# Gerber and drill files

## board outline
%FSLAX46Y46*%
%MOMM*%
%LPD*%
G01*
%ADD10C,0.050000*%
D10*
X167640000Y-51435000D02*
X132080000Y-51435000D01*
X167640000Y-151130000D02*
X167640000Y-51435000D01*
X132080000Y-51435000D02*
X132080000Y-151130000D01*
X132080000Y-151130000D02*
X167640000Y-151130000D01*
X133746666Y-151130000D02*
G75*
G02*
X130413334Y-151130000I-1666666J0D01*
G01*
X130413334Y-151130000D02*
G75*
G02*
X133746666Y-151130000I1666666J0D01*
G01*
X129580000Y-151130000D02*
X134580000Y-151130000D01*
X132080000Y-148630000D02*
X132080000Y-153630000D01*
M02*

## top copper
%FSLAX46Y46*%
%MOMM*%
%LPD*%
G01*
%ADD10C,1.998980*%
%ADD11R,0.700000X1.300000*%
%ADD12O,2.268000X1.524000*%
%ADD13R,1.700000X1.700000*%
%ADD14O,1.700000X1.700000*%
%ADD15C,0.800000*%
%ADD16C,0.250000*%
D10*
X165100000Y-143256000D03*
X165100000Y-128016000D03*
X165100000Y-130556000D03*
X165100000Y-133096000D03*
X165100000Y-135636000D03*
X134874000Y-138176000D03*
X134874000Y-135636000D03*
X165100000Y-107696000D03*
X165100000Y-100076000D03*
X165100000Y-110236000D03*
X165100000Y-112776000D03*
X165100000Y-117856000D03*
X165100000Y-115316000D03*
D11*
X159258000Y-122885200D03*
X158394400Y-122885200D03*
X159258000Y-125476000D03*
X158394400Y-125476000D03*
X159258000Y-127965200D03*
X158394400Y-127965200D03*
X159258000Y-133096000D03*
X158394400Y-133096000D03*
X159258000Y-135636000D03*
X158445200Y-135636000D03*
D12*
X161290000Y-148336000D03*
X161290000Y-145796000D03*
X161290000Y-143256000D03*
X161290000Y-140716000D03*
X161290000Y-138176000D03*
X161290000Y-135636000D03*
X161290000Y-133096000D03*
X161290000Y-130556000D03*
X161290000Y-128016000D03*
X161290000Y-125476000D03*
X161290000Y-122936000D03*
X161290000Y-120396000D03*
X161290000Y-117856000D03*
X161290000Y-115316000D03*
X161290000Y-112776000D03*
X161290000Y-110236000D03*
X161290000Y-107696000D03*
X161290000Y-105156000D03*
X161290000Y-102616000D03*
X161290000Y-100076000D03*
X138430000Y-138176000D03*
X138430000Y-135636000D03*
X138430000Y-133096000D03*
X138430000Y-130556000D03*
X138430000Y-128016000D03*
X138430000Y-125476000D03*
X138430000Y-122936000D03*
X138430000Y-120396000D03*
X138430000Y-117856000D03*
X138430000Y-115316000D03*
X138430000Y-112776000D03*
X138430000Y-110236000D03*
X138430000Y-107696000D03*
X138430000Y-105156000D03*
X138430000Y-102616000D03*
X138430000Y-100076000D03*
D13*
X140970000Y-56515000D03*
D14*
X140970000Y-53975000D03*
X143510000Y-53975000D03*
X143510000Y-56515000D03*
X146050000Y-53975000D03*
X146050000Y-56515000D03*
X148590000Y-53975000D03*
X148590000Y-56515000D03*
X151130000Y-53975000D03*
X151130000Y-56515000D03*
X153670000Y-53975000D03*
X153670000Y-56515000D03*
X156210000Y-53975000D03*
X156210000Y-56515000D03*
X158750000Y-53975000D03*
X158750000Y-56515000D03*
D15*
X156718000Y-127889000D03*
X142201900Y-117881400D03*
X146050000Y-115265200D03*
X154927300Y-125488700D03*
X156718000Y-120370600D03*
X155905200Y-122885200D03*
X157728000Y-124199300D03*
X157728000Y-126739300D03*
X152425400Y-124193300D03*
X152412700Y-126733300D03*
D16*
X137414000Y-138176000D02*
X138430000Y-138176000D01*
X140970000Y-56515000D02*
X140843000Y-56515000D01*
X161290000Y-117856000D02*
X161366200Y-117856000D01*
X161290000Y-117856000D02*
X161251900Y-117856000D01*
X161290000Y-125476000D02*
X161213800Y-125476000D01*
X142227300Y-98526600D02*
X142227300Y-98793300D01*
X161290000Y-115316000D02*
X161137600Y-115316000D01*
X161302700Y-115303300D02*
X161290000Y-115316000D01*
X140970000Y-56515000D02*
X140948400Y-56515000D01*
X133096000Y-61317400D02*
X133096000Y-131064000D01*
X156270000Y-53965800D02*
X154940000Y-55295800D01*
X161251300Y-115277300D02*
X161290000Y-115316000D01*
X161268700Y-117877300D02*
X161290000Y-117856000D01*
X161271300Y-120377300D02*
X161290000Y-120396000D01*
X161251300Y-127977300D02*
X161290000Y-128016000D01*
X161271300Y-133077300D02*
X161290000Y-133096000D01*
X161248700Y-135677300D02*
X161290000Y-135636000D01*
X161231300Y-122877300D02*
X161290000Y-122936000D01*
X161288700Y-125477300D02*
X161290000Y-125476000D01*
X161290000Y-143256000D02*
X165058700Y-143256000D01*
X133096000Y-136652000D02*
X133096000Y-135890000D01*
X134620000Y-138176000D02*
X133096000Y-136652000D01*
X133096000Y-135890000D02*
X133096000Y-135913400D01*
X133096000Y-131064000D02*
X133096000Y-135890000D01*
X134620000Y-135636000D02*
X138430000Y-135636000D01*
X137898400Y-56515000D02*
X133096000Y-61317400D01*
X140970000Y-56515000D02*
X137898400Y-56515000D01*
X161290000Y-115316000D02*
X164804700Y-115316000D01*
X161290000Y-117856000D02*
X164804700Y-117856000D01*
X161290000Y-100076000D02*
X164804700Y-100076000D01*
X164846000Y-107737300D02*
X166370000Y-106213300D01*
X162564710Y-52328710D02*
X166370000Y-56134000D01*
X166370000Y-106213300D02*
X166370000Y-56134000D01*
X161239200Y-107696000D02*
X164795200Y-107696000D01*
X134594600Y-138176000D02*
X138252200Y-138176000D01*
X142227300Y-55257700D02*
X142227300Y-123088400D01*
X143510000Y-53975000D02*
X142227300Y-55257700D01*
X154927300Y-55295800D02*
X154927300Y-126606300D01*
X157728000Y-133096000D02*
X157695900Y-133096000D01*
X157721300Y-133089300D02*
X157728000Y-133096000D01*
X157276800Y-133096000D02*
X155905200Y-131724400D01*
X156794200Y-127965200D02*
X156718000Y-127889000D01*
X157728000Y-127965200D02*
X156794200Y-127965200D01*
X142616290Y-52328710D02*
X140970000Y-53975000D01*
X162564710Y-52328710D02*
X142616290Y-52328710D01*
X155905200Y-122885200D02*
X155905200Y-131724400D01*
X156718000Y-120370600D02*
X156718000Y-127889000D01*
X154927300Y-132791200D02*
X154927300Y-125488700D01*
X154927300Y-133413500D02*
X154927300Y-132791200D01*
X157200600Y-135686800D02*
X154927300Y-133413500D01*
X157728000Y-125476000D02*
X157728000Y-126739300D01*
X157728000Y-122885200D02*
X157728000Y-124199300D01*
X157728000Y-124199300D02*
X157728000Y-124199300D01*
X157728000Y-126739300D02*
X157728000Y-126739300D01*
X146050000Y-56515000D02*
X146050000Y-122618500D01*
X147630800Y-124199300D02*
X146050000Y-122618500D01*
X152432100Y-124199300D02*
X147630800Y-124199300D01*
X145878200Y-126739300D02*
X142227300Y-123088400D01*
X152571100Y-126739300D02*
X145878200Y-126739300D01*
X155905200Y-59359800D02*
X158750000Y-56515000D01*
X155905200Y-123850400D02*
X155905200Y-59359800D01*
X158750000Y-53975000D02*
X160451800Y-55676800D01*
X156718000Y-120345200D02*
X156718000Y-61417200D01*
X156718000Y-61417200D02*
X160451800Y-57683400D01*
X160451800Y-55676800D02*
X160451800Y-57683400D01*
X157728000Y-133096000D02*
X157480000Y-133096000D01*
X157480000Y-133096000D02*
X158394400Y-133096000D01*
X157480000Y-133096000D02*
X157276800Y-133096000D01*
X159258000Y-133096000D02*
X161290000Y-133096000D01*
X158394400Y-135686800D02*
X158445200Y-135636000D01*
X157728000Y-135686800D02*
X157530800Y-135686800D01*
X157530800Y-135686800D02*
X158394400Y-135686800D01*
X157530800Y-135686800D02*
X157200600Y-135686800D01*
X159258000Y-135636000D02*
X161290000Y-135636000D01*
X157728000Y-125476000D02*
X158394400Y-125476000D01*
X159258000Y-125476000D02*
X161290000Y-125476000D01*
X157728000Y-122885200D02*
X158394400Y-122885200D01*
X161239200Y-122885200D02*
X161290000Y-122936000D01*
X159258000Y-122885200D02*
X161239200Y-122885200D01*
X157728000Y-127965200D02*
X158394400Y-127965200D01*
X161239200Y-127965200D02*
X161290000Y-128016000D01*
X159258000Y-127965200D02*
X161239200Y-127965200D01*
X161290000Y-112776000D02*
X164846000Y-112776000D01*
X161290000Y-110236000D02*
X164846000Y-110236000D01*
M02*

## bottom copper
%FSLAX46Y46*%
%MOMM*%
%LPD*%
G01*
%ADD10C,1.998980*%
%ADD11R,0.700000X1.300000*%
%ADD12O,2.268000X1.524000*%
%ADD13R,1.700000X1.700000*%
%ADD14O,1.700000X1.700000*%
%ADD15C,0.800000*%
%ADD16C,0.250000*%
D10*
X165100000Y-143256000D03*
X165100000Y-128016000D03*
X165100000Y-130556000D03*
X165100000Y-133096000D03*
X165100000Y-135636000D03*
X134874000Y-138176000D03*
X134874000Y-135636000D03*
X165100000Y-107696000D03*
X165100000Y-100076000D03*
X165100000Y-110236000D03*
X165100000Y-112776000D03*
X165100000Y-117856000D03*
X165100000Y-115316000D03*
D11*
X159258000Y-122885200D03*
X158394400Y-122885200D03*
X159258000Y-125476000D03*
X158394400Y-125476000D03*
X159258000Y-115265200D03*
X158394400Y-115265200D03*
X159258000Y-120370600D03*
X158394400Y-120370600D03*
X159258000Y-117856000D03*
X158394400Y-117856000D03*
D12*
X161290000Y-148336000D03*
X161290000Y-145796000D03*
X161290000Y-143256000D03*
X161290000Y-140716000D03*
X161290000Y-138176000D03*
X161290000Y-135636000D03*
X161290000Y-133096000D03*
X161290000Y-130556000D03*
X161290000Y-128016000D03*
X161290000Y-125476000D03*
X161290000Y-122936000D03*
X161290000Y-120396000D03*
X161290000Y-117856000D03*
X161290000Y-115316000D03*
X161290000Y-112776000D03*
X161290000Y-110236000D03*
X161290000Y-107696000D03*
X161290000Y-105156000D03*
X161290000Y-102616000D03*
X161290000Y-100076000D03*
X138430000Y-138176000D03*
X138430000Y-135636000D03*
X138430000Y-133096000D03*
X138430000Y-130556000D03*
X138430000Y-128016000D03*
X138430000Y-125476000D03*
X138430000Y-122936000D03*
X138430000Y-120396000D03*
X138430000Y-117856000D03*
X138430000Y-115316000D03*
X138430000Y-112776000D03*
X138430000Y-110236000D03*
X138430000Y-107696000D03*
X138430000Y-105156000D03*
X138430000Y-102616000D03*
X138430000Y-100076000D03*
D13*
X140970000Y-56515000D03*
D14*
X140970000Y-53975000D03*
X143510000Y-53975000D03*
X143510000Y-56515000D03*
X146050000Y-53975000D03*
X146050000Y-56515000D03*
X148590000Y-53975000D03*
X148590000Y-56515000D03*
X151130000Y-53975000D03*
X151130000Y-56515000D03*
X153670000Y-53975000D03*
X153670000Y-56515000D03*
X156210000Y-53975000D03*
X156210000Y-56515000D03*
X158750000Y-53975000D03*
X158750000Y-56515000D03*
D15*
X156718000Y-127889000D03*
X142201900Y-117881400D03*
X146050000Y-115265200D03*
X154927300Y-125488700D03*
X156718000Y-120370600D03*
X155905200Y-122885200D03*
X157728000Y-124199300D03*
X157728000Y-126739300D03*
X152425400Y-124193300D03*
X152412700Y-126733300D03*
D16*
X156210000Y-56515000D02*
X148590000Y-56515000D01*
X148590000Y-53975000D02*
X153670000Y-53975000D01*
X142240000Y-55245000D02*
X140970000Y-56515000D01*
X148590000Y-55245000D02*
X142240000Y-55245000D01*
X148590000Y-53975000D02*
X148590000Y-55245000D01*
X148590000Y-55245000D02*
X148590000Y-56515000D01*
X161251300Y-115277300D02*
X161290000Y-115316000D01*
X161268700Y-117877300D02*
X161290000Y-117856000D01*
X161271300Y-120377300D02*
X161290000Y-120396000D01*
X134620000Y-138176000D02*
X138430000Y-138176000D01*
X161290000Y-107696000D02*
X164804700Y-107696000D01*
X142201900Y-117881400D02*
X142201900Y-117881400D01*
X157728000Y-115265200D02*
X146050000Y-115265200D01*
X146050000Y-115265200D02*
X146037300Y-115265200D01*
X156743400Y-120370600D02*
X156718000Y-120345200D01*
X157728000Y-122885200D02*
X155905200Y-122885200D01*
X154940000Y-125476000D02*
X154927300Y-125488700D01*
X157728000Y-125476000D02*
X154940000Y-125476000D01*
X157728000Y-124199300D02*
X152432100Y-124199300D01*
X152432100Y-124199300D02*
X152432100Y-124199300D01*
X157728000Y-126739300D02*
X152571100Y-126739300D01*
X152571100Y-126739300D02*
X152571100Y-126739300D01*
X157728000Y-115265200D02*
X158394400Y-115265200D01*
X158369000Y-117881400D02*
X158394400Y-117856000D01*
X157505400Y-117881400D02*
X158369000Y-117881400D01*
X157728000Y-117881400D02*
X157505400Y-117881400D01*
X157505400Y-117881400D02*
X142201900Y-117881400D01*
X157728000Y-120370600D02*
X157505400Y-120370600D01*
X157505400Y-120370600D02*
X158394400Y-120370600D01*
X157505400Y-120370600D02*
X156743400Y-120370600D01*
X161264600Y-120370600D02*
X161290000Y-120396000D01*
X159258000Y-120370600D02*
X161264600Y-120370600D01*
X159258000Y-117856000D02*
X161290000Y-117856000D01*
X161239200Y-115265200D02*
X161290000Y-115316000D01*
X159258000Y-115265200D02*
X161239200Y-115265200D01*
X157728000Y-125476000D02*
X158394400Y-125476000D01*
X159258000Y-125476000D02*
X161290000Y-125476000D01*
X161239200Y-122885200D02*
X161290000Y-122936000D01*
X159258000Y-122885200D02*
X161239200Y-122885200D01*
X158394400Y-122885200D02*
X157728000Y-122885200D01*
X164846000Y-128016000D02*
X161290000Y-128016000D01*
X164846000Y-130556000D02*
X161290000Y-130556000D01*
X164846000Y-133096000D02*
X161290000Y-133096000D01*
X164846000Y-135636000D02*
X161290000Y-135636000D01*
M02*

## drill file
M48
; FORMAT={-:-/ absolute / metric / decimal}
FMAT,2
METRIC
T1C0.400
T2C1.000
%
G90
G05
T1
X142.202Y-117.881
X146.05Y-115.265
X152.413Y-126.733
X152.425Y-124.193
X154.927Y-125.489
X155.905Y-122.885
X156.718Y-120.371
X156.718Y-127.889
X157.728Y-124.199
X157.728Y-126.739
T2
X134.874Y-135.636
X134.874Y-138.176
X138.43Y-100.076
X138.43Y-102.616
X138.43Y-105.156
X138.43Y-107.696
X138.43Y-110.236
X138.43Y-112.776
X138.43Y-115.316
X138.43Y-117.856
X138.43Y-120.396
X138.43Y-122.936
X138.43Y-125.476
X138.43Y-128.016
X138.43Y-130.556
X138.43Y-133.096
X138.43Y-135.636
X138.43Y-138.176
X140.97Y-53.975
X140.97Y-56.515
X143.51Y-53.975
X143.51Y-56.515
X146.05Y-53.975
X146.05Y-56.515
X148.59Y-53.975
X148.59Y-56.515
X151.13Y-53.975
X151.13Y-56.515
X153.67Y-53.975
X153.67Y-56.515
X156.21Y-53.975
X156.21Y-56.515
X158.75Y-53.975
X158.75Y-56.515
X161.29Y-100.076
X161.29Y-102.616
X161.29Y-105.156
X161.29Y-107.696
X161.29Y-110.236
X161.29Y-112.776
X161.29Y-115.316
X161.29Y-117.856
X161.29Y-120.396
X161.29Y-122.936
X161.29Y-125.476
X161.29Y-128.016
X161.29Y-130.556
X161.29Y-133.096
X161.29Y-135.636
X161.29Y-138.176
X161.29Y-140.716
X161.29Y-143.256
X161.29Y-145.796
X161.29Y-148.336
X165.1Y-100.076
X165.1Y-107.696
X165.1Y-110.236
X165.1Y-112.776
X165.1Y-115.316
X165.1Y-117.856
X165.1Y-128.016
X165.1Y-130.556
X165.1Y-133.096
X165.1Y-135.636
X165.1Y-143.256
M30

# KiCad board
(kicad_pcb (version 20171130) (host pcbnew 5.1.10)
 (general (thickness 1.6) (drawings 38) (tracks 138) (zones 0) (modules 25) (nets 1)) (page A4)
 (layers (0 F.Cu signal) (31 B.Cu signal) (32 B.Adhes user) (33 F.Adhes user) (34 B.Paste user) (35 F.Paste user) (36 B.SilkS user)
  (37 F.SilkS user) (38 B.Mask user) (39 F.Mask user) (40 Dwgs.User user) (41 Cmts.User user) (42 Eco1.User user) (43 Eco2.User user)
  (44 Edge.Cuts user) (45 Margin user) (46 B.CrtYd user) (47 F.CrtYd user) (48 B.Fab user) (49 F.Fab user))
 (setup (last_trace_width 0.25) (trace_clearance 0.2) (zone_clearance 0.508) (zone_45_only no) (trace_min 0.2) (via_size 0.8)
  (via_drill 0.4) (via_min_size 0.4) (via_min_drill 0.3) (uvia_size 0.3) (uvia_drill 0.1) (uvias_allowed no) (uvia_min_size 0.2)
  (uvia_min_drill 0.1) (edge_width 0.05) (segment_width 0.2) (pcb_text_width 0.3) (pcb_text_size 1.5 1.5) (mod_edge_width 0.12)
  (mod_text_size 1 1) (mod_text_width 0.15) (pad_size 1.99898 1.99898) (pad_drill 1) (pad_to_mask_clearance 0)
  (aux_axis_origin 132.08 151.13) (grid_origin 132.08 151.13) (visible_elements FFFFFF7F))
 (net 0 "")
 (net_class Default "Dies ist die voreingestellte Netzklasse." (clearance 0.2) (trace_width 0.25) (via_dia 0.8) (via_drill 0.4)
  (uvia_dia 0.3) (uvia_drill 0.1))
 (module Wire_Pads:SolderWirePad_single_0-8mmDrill (layer F.Cu) (at 165.1 143.256)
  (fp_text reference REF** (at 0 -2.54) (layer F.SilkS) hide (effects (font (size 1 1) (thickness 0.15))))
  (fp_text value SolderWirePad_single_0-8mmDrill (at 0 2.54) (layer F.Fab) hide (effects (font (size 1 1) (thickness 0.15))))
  (pad 1 thru_hole circle (at 0 0) (size 1.99898 1.99898) (drill 1) (layers *.Cu *.Mask)))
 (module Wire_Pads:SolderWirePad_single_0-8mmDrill (layer F.Cu) (at 165.1 128.016)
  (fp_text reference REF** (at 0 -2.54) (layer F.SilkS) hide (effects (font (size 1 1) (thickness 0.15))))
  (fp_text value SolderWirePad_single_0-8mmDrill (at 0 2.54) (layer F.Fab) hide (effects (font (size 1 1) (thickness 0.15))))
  (pad 1 thru_hole circle (at 0 0) (size 1.99898 1.99898) (drill 1) (layers *.Cu *.Mask)))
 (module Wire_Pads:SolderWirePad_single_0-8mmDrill (layer F.Cu) (at 165.1 130.556)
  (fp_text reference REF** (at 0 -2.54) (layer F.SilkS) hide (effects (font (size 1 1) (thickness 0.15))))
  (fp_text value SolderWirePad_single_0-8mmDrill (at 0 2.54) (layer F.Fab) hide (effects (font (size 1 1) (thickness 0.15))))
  (pad 1 thru_hole circle (at 0 0) (size 1.99898 1.99898) (drill 1) (layers *.Cu *.Mask)))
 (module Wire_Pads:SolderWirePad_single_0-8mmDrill (layer F.Cu) (at 165.1 133.096)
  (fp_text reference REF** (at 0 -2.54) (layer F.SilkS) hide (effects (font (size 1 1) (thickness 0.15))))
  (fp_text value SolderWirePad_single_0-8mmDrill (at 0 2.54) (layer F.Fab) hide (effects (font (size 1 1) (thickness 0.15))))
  (pad 1 thru_hole circle (at 0 0) (size 1.99898 1.99898) (drill 1) (layers *.Cu *.Mask)))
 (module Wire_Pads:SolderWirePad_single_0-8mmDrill (layer F.Cu) (at 165.1 135.636)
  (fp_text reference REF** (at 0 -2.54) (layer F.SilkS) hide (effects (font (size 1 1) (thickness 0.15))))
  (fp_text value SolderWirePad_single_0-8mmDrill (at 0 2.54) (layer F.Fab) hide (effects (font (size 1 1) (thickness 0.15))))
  (pad 1 thru_hole circle (at 0 0) (size 1.99898 1.99898) (drill 1) (layers *.Cu *.Mask)))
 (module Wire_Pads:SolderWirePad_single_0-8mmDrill (layer F.Cu) (at 134.874 138.176)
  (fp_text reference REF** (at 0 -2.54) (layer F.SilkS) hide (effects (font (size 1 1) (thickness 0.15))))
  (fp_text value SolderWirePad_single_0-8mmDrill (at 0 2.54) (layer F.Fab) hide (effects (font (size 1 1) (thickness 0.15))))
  (pad 1 thru_hole circle (at 0 0) (size 1.99898 1.99898) (drill 1) (layers *.Cu *.Mask)))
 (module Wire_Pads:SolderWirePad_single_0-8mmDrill (layer F.Cu) (at 134.874 135.636)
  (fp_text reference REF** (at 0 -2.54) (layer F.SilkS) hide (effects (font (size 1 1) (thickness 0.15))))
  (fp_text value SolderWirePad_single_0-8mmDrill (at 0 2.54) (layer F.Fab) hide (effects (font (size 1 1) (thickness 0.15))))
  (pad 1 thru_hole circle (at 0 0) (size 1.99898 1.99898) (drill 1) (layers *.Cu *.Mask)))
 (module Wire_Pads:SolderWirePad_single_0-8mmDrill (layer F.Cu) (at 165.1 107.696)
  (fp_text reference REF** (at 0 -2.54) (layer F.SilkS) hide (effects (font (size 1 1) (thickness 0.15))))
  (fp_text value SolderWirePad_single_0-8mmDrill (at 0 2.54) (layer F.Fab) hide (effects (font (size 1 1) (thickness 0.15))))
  (pad 1 thru_hole circle (at 0 0) (size 1.99898 1.99898) (drill 1) (layers *.Cu *.Mask)))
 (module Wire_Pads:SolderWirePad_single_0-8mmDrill (layer F.Cu) (at 165.1 100.076)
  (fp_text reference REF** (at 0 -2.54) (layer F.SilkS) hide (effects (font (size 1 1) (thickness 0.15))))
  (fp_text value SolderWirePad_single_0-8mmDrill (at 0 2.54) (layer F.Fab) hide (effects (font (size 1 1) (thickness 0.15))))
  (pad 1 thru_hole circle (at 0 0) (size 1.99898 1.99898) (drill 1) (layers *.Cu *.Mask)))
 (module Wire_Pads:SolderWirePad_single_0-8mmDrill (layer F.Cu) (at 165.1 110.236)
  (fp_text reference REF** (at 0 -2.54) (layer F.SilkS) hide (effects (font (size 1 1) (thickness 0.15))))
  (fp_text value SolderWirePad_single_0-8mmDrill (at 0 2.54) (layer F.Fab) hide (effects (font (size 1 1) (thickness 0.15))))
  (pad 1 thru_hole circle (at 0 0) (size 1.99898 1.99898) (drill 1) (layers *.Cu *.Mask)))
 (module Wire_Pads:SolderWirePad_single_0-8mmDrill (layer F.Cu) (at 165.1 112.776)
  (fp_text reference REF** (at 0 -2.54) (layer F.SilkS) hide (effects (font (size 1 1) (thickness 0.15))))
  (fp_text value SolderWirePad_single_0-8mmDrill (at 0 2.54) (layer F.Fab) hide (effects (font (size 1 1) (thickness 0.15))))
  (pad 1 thru_hole circle (at 0 0) (size 1.99898 1.99898) (drill 1) (layers *.Cu *.Mask)))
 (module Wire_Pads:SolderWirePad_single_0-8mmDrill (layer F.Cu) (at 165.1 117.856)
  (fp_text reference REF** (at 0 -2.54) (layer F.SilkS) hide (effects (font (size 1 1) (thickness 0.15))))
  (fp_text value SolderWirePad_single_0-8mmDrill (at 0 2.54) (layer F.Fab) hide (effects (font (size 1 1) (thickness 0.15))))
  (pad 1 thru_hole circle (at 0 0) (size 1.99898 1.99898) (drill 1) (layers *.Cu *.Mask)))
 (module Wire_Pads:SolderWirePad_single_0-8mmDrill (layer F.Cu) (at 165.1 115.316)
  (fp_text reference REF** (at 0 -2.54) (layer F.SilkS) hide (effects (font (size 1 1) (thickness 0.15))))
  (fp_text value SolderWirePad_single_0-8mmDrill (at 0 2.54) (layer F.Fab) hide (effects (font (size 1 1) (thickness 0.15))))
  (pad 1 thru_hole circle (at 0 0) (size 1.99898 1.99898) (drill 1) (layers *.Cu *.Mask)))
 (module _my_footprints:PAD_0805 (layer B.Cu) (at 158.8262 122.8852)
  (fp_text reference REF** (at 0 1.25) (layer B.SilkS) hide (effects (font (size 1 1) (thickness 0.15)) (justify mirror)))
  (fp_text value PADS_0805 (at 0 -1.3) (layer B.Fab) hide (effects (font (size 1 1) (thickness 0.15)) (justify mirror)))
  (pad 2 smd rect (at 0.4318 0) (size 0.7 1.3) (layers B.Cu B.Paste B.Mask))
  (pad 1 smd rect (at -0.4318 0) (size 0.7 1.3) (layers B.Cu B.Paste B.Mask)))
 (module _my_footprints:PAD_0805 (layer B.Cu) (at 158.8262 125.476)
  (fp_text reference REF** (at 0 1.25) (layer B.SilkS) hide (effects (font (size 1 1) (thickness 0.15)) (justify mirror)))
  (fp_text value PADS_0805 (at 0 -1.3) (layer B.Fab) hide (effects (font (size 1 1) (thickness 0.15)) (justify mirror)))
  (pad 2 smd rect (at 0.4318 0) (size 0.7 1.3) (layers B.Cu B.Paste B.Mask))
  (pad 1 smd rect (at -0.4318 0) (size 0.7 1.3) (layers B.Cu B.Paste B.Mask)))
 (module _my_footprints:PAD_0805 (layer B.Cu) (at 158.8262 115.2652)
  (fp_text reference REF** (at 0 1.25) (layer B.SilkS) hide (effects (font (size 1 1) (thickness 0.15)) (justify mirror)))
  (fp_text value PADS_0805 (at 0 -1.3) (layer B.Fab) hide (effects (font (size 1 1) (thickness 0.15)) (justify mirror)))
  (pad 2 smd rect (at 0.4318 0) (size 0.7 1.3) (layers B.Cu B.Paste B.Mask))
  (pad 1 smd rect (at -0.4318 0) (size 0.7 1.3) (layers B.Cu B.Paste B.Mask)))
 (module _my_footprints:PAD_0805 (layer B.Cu) (at 158.8262 120.3706)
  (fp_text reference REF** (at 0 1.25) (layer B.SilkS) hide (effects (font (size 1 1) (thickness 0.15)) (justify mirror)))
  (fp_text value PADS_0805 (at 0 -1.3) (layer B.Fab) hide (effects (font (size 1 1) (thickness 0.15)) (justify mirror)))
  (pad 2 smd rect (at 0.4318 0) (size 0.7 1.3) (layers B.Cu B.Paste B.Mask))
  (pad 1 smd rect (at -0.4318 0) (size 0.7 1.3) (layers B.Cu B.Paste B.Mask)))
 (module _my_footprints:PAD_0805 (layer B.Cu) (at 158.8262 117.856)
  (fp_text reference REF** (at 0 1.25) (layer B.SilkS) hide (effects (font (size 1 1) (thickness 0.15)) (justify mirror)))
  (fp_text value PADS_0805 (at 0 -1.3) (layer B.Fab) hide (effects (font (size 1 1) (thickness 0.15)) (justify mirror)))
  (pad 2 smd rect (at 0.4318 0) (size 0.7 1.3) (layers B.Cu B.Paste B.Mask))
  (pad 1 smd rect (at -0.4318 0) (size 0.7 1.3) (layers B.Cu B.Paste B.Mask)))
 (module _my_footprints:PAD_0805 (layer F.Cu) (at 158.8262 122.8852)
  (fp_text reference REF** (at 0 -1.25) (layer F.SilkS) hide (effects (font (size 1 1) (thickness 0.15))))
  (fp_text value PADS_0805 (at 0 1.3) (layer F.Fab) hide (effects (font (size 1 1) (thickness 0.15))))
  (pad 2 smd rect (at 0.4318 0) (size 0.7 1.3) (layers F.Cu F.Paste F.Mask))
  (pad 1 smd rect (at -0.4318 0) (size 0.7 1.3) (layers F.Cu F.Paste F.Mask)))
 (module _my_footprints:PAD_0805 (layer F.Cu) (at 158.8262 125.476)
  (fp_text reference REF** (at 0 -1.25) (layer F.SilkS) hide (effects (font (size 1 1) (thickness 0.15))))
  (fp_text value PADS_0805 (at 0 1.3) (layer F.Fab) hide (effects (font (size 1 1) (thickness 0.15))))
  (pad 2 smd rect (at 0.4318 0) (size 0.7 1.3) (layers F.Cu F.Paste F.Mask))
  (pad 1 smd rect (at -0.4318 0) (size 0.7 1.3) (layers F.Cu F.Paste F.Mask)))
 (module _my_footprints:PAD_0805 (layer F.Cu) (at 158.8262 127.9652)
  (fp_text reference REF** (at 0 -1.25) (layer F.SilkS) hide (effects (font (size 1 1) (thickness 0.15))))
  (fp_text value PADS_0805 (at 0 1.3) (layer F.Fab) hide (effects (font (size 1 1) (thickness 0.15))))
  (pad 2 smd rect (at 0.4318 0) (size 0.7 1.3) (layers F.Cu F.Paste F.Mask))
  (pad 1 smd rect (at -0.4318 0) (size 0.7 1.3) (layers F.Cu F.Paste F.Mask)))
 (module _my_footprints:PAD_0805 (layer F.Cu) (at 158.8262 133.096)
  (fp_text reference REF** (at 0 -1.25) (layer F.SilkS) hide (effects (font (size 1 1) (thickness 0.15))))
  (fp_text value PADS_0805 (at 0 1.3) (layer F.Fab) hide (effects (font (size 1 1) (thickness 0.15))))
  (pad 2 smd rect (at 0.4318 0) (size 0.7 1.3) (layers F.Cu F.Paste F.Mask))
  (pad 1 smd rect (at -0.4318 0) (size 0.7 1.3) (layers F.Cu F.Paste F.Mask)))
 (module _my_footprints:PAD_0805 (layer F.Cu) (at 158.8516 135.636)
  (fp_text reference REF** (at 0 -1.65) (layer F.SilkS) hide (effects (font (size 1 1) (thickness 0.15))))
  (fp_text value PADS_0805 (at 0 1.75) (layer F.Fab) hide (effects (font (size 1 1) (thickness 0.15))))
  (pad 2 smd rect (at 0.4064 0) (size 0.7 1.3) (layers F.Cu F.Paste F.Mask))
  (pad 1 smd rect (at -0.4064 0) (size 0.7 1.3) (layers F.Cu F.Paste F.Mask)))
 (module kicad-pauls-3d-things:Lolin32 (layer F.Cu) (at 147.32 110.236)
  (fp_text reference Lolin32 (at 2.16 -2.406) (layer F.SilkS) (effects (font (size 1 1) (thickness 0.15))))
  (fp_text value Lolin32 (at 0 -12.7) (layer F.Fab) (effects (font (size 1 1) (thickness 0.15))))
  (pad 15 thru_hole oval (at 13.97 38.1) (size 2.268 1.524) (drill 1) (layers *.Cu *.Mask))
  (pad 2 thru_hole oval (at 13.97 35.56) (size 2.268 1.524) (drill 1) (layers *.Cu *.Mask))
  (pad G thru_hole oval (at 13.97 33.02) (size 2.268 1.524) (drill 1) (layers *.Cu *.Mask))
  (pad 0 thru_hole oval (at 13.97 30.48) (size 2.268 1.524) (drill 1) (layers *.Cu *.Mask))
  (pad 4 thru_hole oval (at 13.97 27.94) (size 2.268 1.524) (drill 1) (layers *.Cu *.Mask))
  (pad 16 thru_hole oval (at 13.97 25.4) (size 2.268 1.524) (drill 1) (layers *.Cu *.Mask))
  (pad 17 thru_hole oval (at 13.97 22.86) (size 2.268 1.524) (drill 1) (layers *.Cu *.Mask))
  (pad 3.3V thru_hole oval (at 13.97 20.32) (size 2.268 1.524) (drill 1) (layers *.Cu *.Mask))
  (pad 5 thru_hole oval (at 13.97 17.78) (size 2.268 1.524) (drill 1) (layers *.Cu *.Mask))
  (pad 18 thru_hole oval (at 13.97 15.24) (size 2.268 1.524) (drill 1) (layers *.Cu *.Mask))
  (pad 23 thru_hole oval (at 13.97 12.7) (size 2.268 1.524) (drill 1) (layers *.Cu *.Mask))
  (pad 19 thru_hole oval (at 13.97 10.16) (size 2.268 1.524) (drill 1) (layers *.Cu *.Mask))
  (pad G thru_hole oval (at 13.97 7.62) (size 2.268 1.524) (drill 1) (layers *.Cu *.Mask))
  (pad G thru_hole oval (at 13.97 5.08) (size 2.268 1.524) (drill 1) (layers *.Cu *.Mask))
  (pad 21 thru_hole oval (at 13.97 2.54) (size 2.268 1.524) (drill 1) (layers *.Cu *.Mask))
  (pad 22 thru_hole oval (at 13.97 0) (size 2.268 1.524) (drill 1) (layers *.Cu *.Mask))
  (pad 3.3V thru_hole oval (at 13.97 -2.54) (size 2.268 1.524) (drill 1) (layers *.Cu *.Mask))
  (pad 3 thru_hole oval (at 13.97 -5.08) (size 2.268 1.524) (drill 1) (layers *.Cu *.Mask))
  (pad 1 thru_hole oval (at 13.97 -7.62) (size 2.268 1.524) (drill 1) (layers *.Cu *.Mask))
  (pad G thru_hole oval (at 13.97 -10.16) (size 2.268 1.524) (drill 1) (layers *.Cu *.Mask))
  (pad G thru_hole oval (at -8.89 27.94) (size 2.268 1.524) (drill 1) (layers *.Cu *.Mask))
  (pad 5V thru_hole oval (at -8.89 25.4) (size 2.268 1.524) (drill 1) (layers *.Cu *.Mask))
  (pad 13 thru_hole oval (at -8.89 22.86) (size 2.268 1.524) (drill 1) (layers *.Cu *.Mask))
  (pad 12 thru_hole oval (at -8.89 20.32) (size 2.268 1.524) (drill 1) (layers *.Cu *.Mask))
  (pad 14 thru_hole oval (at -8.89 17.78) (size 2.268 1.524) (drill 1) (layers *.Cu *.Mask))
  (pad 27 thru_hole oval (at -8.89 15.24) (size 2.268 1.524) (drill 1) (layers *.Cu *.Mask))
  (pad 26 thru_hole oval (at -8.89 12.7) (size 2.268 1.524) (drill 1) (layers *.Cu *.Mask))
  (pad 25 thru_hole oval (at -8.89 10.16) (size 2.268 1.524) (drill 1) (layers *.Cu *.Mask))
  (pad 35 thru_hole oval (at -8.89 7.62) (size 2.268 1.524) (drill 1) (layers *.Cu *.Mask))
  (pad 34 thru_hole oval (at -8.89 5.08) (size 2.268 1.524) (drill 1) (layers *.Cu *.Mask))
  (pad 33 thru_hole oval (at -8.89 2.54) (size 2.268 1.524) (drill 1) (layers *.Cu *.Mask))
  (pad 32 thru_hole oval (at -8.89 0) (size 2.268 1.524) (drill 1) (layers *.Cu *.Mask))
  (pad 39 thru_hole oval (at -8.89 -2.54) (size 2.268 1.524) (drill 1) (layers *.Cu *.Mask))
  (pad 36 thru_hole oval (at -8.89 -5.08) (size 2.268 1.524) (drill 1) (layers *.Cu *.Mask))
  (pad EN thru_hole oval (at -8.89 -7.62) (size 2.268 1.524) (drill 1) (layers *.Cu *.Mask))
  (pad 3.3V thru_hole oval (at -8.89 -10.16) (size 2.268 1.524) (drill 1) (layers *.Cu *.Mask)))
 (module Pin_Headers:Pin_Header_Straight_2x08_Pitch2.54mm (layer B.Cu) (at 140.97 53.975 270)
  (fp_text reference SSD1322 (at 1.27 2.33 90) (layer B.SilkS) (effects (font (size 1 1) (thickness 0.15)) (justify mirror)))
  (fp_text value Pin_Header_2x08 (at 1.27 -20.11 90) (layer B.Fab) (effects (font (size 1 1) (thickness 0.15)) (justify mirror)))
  (pad 1 thru_hole rect (at 2.54 0 270) (size 1.7 1.7) (drill 1) (layers *.Cu *.Mask))
  (pad 2 thru_hole oval (at 0 0 270) (size 1.7 1.7) (drill 1) (layers *.Cu *.Mask))
  (pad 4 thru_hole oval (at 0 -2.54 270) (size 1.7 1.7) (drill 1) (layers *.Cu *.Mask))
  (pad 3 thru_hole oval (at 2.54 -2.54 270) (size 1.7 1.7) (drill 1) (layers *.Cu *.Mask))
  (pad 6 thru_hole oval (at 0 -5.08 270) (size 1.7 1.7) (drill 1) (layers *.Cu *.Mask))
  (pad 5 thru_hole oval (at 2.54 -5.08 270) (size 1.7 1.7) (drill 1) (layers *.Cu *.Mask))
  (pad 8 thru_hole oval (at 0 -7.62 270) (size 1.7 1.7) (drill 1) (layers *.Cu *.Mask))
  (pad 7 thru_hole oval (at 2.54 -7.62 270) (size 1.7 1.7) (drill 1) (layers *.Cu *.Mask))
  (pad 10 thru_hole oval (at 0 -10.16 270) (size 1.7 1.7) (drill 1) (layers *.Cu *.Mask))
  (pad 9 thru_hole oval (at 2.54 -10.16 270) (size 1.7 1.7) (drill 1) (layers *.Cu *.Mask))
  (pad 12 thru_hole oval (at 0 -12.7 270) (size 1.7 1.7) (drill 1) (layers *.Cu *.Mask))
  (pad 11 thru_hole oval (at 2.54 -12.7 270) (size 1.7 1.7) (drill 1) (layers *.Cu *.Mask))
  (pad 14 thru_hole oval (at 0 -15.24 270) (size 1.7 1.7) (drill 1) (layers *.Cu *.Mask))
  (pad 13 thru_hole oval (at 2.54 -15.24 270) (size 1.7 1.7) (drill 1) (layers *.Cu *.Mask))
  (pad 16 thru_hole oval (at 0 -17.78 270) (size 1.7 1.7) (drill 1) (layers *.Cu *.Mask))
  (pad 15 thru_hole oval (at 2.54 -17.78 270) (size 1.7 1.7) (drill 1) (layers *.Cu *.Mask)))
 (gr_line (start 167.64 51.435) (end 132.08 51.435) (layer Edge.Cuts) (width 0.05))
 (gr_line (start 167.64 151.13) (end 167.64 51.435) (layer Edge.Cuts) (width 0.05))
 (gr_line (start 132.08 51.435) (end 132.08 151.13) (layer Edge.Cuts) (width 0.05))
 (gr_line (start 132.08 151.13) (end 167.64 151.13) (layer Edge.Cuts) (width 0.05))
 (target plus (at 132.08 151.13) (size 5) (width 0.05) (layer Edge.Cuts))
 (segment (start 156.21 56.515) (end 148.59 56.515) (width 0.25) (layer B.Cu) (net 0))
 (segment (start 148.59 53.975) (end 153.67 53.975) (width 0.25) (layer B.Cu) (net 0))
 (segment (start 142.24 55.245) (end 140.97 56.515) (width 0.25) (layer B.Cu) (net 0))
 (segment (start 148.59 55.245) (end 142.24 55.245) (width 0.25) (layer B.Cu) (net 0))
 (segment (start 148.59 53.975) (end 148.59 55.245) (width 0.25) (layer B.Cu) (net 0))
 (segment (start 148.59 55.245) (end 148.59 56.515) (width 0.25) (layer B.Cu) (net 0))
 (segment (start 137.414 138.176) (end 138.43 138.176) (width 0.25) (layer F.Cu) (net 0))
 (segment (start 140.97 56.515) (end 140.843 56.515) (width 0.25) (layer F.Cu) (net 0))
 (segment (start 161.29 117.856) (end 161.3662 117.856) (width 0.25) (layer F.Cu) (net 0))
 (segment (start 161.29 117.856) (end 161.2519 117.856) (width 0.25) (layer F.Cu) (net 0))
 (segment (start 161.29 125.476) (end 161.2138 125.476) (width 0.25) (layer F.Cu) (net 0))
 (segment (start 142.2273 98.5266) (end 142.2273 98.7933) (width 0.25) (layer F.Cu) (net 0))
 (segment (start 161.29 115.316) (end 161.1376 115.316) (width 0.25) (layer F.Cu) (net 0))
 (segment (start 161.3027 115.3033) (end 161.29 115.316) (width 0.25) (layer F.Cu) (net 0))
 (segment (start 140.97 56.515) (end 140.9484 56.515) (width 0.25) (layer F.Cu) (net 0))
 (segment (start 133.096 61.3174) (end 133.096 131.064) (width 0.25) (layer F.Cu) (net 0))
 (segment (start 156.27 53.9658) (end 154.94 55.2958) (width 0.25) (layer F.Cu) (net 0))
 (segment (start 161.2513 115.2773) (end 161.29 115.316) (width 0.25) (layer F.Cu) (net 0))
 (segment (start 161.2687 117.8773) (end 161.29 117.856) (width 0.25) (layer F.Cu) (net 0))
 (segment (start 161.2713 120.3773) (end 161.29 120.396) (width 0.25) (layer F.Cu) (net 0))
 (segment (start 161.2513 127.9773) (end 161.29 128.016) (width 0.25) (layer F.Cu) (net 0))
 (segment (start 161.2713 133.0773) (end 161.29 133.096) (width 0.25) (layer F.Cu) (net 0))
 (segment (start 161.2487 135.6773) (end 161.29 135.636) (width 0.25) (layer F.Cu) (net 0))
 (segment (start 161.2313 122.8773) (end 161.29 122.936) (width 0.25) (layer F.Cu) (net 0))
 (segment (start 161.2887 125.4773) (end 161.29 125.476) (width 0.25) (layer F.Cu) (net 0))
 (segment (start 161.2513 115.2773) (end 161.29 115.316) (width 0.25) (layer B.Cu) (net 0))
 (segment (start 161.2687 117.8773) (end 161.29 117.856) (width 0.25) (layer B.Cu) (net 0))
 (segment (start 161.2713 120.3773) (end 161.29 120.396) (width 0.25) (layer B.Cu) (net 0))
 (segment (start 161.29 143.256) (end 165.0587 143.256) (width 0.25) (layer F.Cu) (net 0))
 (segment (start 133.096 136.652) (end 133.096 135.89) (width 0.25) (layer F.Cu) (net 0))
 (segment (start 134.62 138.176) (end 133.096 136.652) (width 0.25) (layer F.Cu) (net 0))
 (segment (start 133.096 135.89) (end 133.096 135.9134) (width 0.25) (layer F.Cu) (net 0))
 (segment (start 133.096 131.064) (end 133.096 135.89) (width 0.25) (layer F.Cu) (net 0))
 (segment (start 134.62 135.636) (end 138.43 135.636) (width 0.25) (layer F.Cu) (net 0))
 (segment (start 137.8984 56.515) (end 133.096 61.3174) (width 0.25) (layer F.Cu) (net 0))
 (segment (start 140.97 56.515) (end 137.8984 56.515) (width 0.25) (layer F.Cu) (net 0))
 (segment (start 161.29 115.316) (end 164.8047 115.316) (width 0.25) (layer F.Cu) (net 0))
 (segment (start 161.29 117.856) (end 164.8047 117.856) (width 0.25) (layer F.Cu) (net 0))
 (segment (start 161.29 100.076) (end 164.8047 100.076) (width 0.25) (layer F.Cu) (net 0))
 (segment (start 164.846 107.7373) (end 166.37 106.2133) (width 0.25) (layer F.Cu) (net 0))
 (segment (start 162.56471 52.32871) (end 166.37 56.134) (width 0.25) (layer F.Cu) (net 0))
 (segment (start 166.37 106.2133) (end 166.37 56.134) (width 0.25) (layer F.Cu) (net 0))
 (segment (start 134.62 138.176) (end 138.43 138.176) (width 0.25) (layer B.Cu) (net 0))
 (segment (start 161.29 107.696) (end 164.8047 107.696) (width 0.25) (layer B.Cu) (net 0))
 (segment (start 161.2392 107.696) (end 164.7952 107.696) (width 0.25) (layer F.Cu) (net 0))
 (segment (start 134.5946 138.176) (end 138.2522 138.176) (width 0.25) (layer F.Cu) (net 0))
 (segment (start 142.2273 55.2577) (end 142.2273 123.0884) (width 0.25) (layer F.Cu) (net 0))
 (segment (start 143.51 53.975) (end 142.2273 55.2577) (width 0.25) (layer F.Cu) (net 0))
 (segment (start 154.9273 55.2958) (end 154.9273 126.6063) (width 0.25) (layer F.Cu) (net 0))
 (segment (start 157.728 133.096) (end 157.6959 133.096) (width 0.25) (layer F.Cu) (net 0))
 (segment (start 157.7213 133.0893) (end 157.728 133.096) (width 0.25) (layer F.Cu) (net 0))
 (via (at 156.718 127.889) (size 0.8) (drill 0.4) (layers F.Cu B.Cu) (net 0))
 (segment (start 157.2768 133.096) (end 155.9052 131.7244) (width 0.25) (layer F.Cu) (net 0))
 (segment (start 156.7942 127.9652) (end 156.718 127.889) (width 0.25) (layer F.Cu) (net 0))
 (segment (start 157.728 127.9652) (end 156.7942 127.9652) (width 0.25) (layer F.Cu) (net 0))
 (segment (start 142.2019 117.8814) (end 142.2019 117.8814) (width 0.25) (layer B.Cu) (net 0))
 (via (at 142.2019 117.8814) (size 0.8) (drill 0.4) (layers F.Cu B.Cu) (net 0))
 (segment (start 157.728 115.2652) (end 146.05 115.2652) (width 0.25) (layer B.Cu) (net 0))
 (segment (start 146.05 115.2652) (end 146.0373 115.2652) (width 0.25) (layer B.Cu) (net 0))
 (via (at 146.05 115.2652) (size 0.8) (drill 0.4) (layers F.Cu B.Cu) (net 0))
 (via (at 154.9273 125.4887) (size 0.8) (drill 0.4) (layers F.Cu B.Cu) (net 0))
 (via (at 156.718 120.3706) (size 0.8) (drill 0.4) (layers F.Cu B.Cu) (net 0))
 (segment (start 156.7434 120.3706) (end 156.718 120.3452) (width 0.25) (layer B.Cu) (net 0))
 (via (at 155.9052 122.8852) (size 0.8) (drill 0.4) (layers F.Cu B.Cu) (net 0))
 (segment (start 142.61629 52.32871) (end 140.97 53.975) (width 0.25) (layer F.Cu) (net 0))
 (segment (start 162.56471 52.32871) (end 142.61629 52.32871) (width 0.25) (layer F.Cu) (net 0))
 (segment (start 157.728 122.8852) (end 155.9052 122.8852) (width 0.25) (layer B.Cu) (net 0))
 (segment (start 154.94 125.476) (end 154.9273 125.4887) (width 0.25) (layer B.Cu) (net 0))
 (segment (start 157.728 125.476) (end 154.94 125.476) (width 0.25) (layer B.Cu) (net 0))
 (segment (start 155.9052 122.8852) (end 155.9052 131.7244) (width 0.25) (layer F.Cu) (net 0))
 (segment (start 156.718 120.3706) (end 156.718 127.889) (width 0.25) (layer F.Cu) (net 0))
 (segment (start 154.9273 132.7912) (end 154.9273 125.4887) (width 0.25) (layer F.Cu) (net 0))
 (segment (start 154.9273 133.4135) (end 154.9273 132.7912) (width 0.25) (layer F.Cu) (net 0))
 (segment (start 157.2006 135.6868) (end 154.9273 133.4135) (width 0.25) (layer F.Cu) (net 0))
 (segment (start 157.728 125.476) (end 157.728 126.7393) (width 0.25) (layer F.Cu) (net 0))
 (segment (start 157.728 122.8852) (end 157.728 124.1993) (width 0.25) (layer F.Cu) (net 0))
 (segment (start 157.728 124.1993) (end 157.728 124.1993) (width 0.25) (layer F.Cu) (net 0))
 (via (at 157.728 124.1993) (size 0.8) (drill 0.4) (layers F.Cu B.Cu) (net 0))
 (segment (start 157.728 126.7393) (end 157.728 126.7393) (width 0.25) (layer F.Cu) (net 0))
 (via (at 157.728 126.7393) (size 0.8) (drill 0.4) (layers F.Cu B.Cu) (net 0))
 (segment (start 157.728 124.1993) (end 152.4321 124.1993) (width 0.25) (layer B.Cu) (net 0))
 (segment (start 152.4321 124.1993) (end 152.4321 124.1993) (width 0.25) (layer B.Cu) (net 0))
 (via (at 152.4254 124.1933) (size 0.8) (drill 0.4) (layers F.Cu B.Cu) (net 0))
 (segment (start 146.05 56.515) (end 146.05 122.6185) (width 0.25) (layer F.Cu) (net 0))
 (segment (start 147.6308 124.1993) (end 146.05 122.6185) (width 0.25) (layer F.Cu) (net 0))
 (segment (start 152.4321 124.1993) (end 147.6308 124.1993) (width 0.25) (layer F.Cu) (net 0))
 (segment (start 157.728 126.7393) (end 152.5711 126.7393) (width 0.25) (layer B.Cu) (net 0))
 (segment (start 152.5711 126.7393) (end 152.5711 126.7393) (width 0.25) (layer B.Cu) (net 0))
 (via (at 152.4127 126.7333) (size 0.8) (drill 0.4) (layers F.Cu B.Cu) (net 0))
 (segment (start 145.8782 126.7393) (end 142.2273 123.0884) (width 0.25) (layer F.Cu) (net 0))
 (segment (start 152.5711 126.7393) (end 145.8782 126.7393) (width 0.25) (layer F.Cu) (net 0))
 (segment (start 155.9052 59.3598) (end 158.75 56.515) (width 0.25) (layer F.Cu) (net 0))
 (segment (start 155.9052 123.8504) (end 155.9052 59.3598) (width 0.25) (layer F.Cu) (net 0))
 (segment (start 158.75 53.975) (end 160.4518 55.6768) (width 0.25) (layer F.Cu) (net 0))
 (segment (start 156.718 120.3452) (end 156.718 61.4172) (width 0.25) (layer F.Cu) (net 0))
 (segment (start 156.718 61.4172) (end 160.4518 57.6834) (width 0.25) (layer F.Cu) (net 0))
 (segment (start 160.4518 55.6768) (end 160.4518 57.6834) (width 0.25) (layer F.Cu) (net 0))
 (segment (start 157.728 133.096) (end 157.48 133.096) (width 0.25) (layer F.Cu) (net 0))
 (segment (start 157.48 133.096) (end 158.3944 133.096) (width 0.25) (layer F.Cu) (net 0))
 (segment (start 157.48 133.096) (end 157.2768 133.096) (width 0.25) (layer F.Cu) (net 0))
 (segment (start 159.258 133.096) (end 161.29 133.096) (width 0.25) (layer F.Cu) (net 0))
 (segment (start 158.3944 135.6868) (end 158.4452 135.636) (width 0.25) (layer F.Cu) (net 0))
 (segment (start 157.728 135.6868) (end 157.5308 135.6868) (width 0.25) (layer F.Cu) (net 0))
 (segment (start 157.5308 135.6868) (end 158.3944 135.6868) (width 0.25) (layer F.Cu) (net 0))
 (segment (start 157.5308 135.6868) (end 157.2006 135.6868) (width 0.25) (layer F.Cu) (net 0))
 (segment (start 159.258 135.636) (end 161.29 135.636) (width 0.25) (layer F.Cu) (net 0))
 (segment (start 157.728 125.476) (end 158.3944 125.476) (width 0.25) (layer F.Cu) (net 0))
 (segment (start 159.258 125.476) (end 161.29 125.476) (width 0.25) (layer F.Cu) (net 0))
 (segment (start 157.728 122.8852) (end 158.3944 122.8852) (width 0.25) (layer F.Cu) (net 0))
 (segment (start 161.2392 122.8852) (end 161.29 122.936) (width 0.25) (layer F.Cu) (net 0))
 (segment (start 159.258 122.8852) (end 161.2392 122.8852) (width 0.25) (layer F.Cu) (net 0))
 (segment (start 157.728 115.2652) (end 158.3944 115.2652) (width 0.25) (layer B.Cu) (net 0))
 (segment (start 158.369 117.8814) (end 158.3944 117.856) (width 0.25) (layer B.Cu) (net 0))
 (segment (start 157.5054 117.8814) (end 158.369 117.8814) (width 0.25) (layer B.Cu) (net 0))
 (segment (start 157.728 117.8814) (end 157.5054 117.8814) (width 0.25) (layer B.Cu) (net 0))
 (segment (start 157.5054 117.8814) (end 142.2019 117.8814) (width 0.25) (layer B.Cu) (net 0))
 (segment (start 157.728 120.3706) (end 157.5054 120.3706) (width 0.25) (layer B.Cu) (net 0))
 (segment (start 157.5054 120.3706) (end 158.3944 120.3706) (width 0.25) (layer B.Cu) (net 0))
 (segment (start 157.5054 120.3706) (end 156.7434 120.3706) (width 0.25) (layer B.Cu) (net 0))
 (segment (start 161.2646 120.3706) (end 161.29 120.396) (width 0.25) (layer B.Cu) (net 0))
 (segment (start 159.258 120.3706) (end 161.2646 120.3706) (width 0.25) (layer B.Cu) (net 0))
 (segment (start 159.258 117.856) (end 161.29 117.856) (width 0.25) (layer B.Cu) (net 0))
 (segment (start 161.2392 115.2652) (end 161.29 115.316) (width 0.25) (layer B.Cu) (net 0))
 (segment (start 159.258 115.2652) (end 161.2392 115.2652) (width 0.25) (layer B.Cu) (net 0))
 (segment (start 157.728 125.476) (end 158.3944 125.476) (width 0.25) (layer B.Cu) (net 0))
 (segment (start 159.258 125.476) (end 161.29 125.476) (width 0.25) (layer B.Cu) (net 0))
 (segment (start 161.2392 122.8852) (end 161.29 122.936) (width 0.25) (layer B.Cu) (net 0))
 (segment (start 159.258 122.8852) (end 161.2392 122.8852) (width 0.25) (layer B.Cu) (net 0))
 (segment (start 158.3944 122.8852) (end 157.728 122.8852) (width 0.25) (layer B.Cu) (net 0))
 (segment (start 157.728 127.9652) (end 158.3944 127.9652) (width 0.25) (layer F.Cu) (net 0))
 (segment (start 161.2392 127.9652) (end 161.29 128.016) (width 0.25) (layer F.Cu) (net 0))
 (segment (start 159.258 127.9652) (end 161.2392 127.9652) (width 0.25) (layer F.Cu) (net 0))
 (segment (start 161.29 112.776) (end 164.846 112.776) (width 0.25) (layer F.Cu) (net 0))
 (segment (start 161.29 110.236) (end 164.846 110.236) (width 0.25) (layer F.Cu) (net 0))
 (segment (start 164.846 128.016) (end 161.29 128.016) (width 0.25) (layer B.Cu) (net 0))
 (segment (start 164.846 130.556) (end 161.29 130.556) (width 0.25) (layer B.Cu) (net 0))
 (segment (start 164.846 133.096) (end 161.29 133.096) (width 0.25) (layer B.Cu) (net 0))
 (segment (start 164.846 135.636) (end 161.29 135.636) (width 0.25) (layer B.Cu) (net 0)))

